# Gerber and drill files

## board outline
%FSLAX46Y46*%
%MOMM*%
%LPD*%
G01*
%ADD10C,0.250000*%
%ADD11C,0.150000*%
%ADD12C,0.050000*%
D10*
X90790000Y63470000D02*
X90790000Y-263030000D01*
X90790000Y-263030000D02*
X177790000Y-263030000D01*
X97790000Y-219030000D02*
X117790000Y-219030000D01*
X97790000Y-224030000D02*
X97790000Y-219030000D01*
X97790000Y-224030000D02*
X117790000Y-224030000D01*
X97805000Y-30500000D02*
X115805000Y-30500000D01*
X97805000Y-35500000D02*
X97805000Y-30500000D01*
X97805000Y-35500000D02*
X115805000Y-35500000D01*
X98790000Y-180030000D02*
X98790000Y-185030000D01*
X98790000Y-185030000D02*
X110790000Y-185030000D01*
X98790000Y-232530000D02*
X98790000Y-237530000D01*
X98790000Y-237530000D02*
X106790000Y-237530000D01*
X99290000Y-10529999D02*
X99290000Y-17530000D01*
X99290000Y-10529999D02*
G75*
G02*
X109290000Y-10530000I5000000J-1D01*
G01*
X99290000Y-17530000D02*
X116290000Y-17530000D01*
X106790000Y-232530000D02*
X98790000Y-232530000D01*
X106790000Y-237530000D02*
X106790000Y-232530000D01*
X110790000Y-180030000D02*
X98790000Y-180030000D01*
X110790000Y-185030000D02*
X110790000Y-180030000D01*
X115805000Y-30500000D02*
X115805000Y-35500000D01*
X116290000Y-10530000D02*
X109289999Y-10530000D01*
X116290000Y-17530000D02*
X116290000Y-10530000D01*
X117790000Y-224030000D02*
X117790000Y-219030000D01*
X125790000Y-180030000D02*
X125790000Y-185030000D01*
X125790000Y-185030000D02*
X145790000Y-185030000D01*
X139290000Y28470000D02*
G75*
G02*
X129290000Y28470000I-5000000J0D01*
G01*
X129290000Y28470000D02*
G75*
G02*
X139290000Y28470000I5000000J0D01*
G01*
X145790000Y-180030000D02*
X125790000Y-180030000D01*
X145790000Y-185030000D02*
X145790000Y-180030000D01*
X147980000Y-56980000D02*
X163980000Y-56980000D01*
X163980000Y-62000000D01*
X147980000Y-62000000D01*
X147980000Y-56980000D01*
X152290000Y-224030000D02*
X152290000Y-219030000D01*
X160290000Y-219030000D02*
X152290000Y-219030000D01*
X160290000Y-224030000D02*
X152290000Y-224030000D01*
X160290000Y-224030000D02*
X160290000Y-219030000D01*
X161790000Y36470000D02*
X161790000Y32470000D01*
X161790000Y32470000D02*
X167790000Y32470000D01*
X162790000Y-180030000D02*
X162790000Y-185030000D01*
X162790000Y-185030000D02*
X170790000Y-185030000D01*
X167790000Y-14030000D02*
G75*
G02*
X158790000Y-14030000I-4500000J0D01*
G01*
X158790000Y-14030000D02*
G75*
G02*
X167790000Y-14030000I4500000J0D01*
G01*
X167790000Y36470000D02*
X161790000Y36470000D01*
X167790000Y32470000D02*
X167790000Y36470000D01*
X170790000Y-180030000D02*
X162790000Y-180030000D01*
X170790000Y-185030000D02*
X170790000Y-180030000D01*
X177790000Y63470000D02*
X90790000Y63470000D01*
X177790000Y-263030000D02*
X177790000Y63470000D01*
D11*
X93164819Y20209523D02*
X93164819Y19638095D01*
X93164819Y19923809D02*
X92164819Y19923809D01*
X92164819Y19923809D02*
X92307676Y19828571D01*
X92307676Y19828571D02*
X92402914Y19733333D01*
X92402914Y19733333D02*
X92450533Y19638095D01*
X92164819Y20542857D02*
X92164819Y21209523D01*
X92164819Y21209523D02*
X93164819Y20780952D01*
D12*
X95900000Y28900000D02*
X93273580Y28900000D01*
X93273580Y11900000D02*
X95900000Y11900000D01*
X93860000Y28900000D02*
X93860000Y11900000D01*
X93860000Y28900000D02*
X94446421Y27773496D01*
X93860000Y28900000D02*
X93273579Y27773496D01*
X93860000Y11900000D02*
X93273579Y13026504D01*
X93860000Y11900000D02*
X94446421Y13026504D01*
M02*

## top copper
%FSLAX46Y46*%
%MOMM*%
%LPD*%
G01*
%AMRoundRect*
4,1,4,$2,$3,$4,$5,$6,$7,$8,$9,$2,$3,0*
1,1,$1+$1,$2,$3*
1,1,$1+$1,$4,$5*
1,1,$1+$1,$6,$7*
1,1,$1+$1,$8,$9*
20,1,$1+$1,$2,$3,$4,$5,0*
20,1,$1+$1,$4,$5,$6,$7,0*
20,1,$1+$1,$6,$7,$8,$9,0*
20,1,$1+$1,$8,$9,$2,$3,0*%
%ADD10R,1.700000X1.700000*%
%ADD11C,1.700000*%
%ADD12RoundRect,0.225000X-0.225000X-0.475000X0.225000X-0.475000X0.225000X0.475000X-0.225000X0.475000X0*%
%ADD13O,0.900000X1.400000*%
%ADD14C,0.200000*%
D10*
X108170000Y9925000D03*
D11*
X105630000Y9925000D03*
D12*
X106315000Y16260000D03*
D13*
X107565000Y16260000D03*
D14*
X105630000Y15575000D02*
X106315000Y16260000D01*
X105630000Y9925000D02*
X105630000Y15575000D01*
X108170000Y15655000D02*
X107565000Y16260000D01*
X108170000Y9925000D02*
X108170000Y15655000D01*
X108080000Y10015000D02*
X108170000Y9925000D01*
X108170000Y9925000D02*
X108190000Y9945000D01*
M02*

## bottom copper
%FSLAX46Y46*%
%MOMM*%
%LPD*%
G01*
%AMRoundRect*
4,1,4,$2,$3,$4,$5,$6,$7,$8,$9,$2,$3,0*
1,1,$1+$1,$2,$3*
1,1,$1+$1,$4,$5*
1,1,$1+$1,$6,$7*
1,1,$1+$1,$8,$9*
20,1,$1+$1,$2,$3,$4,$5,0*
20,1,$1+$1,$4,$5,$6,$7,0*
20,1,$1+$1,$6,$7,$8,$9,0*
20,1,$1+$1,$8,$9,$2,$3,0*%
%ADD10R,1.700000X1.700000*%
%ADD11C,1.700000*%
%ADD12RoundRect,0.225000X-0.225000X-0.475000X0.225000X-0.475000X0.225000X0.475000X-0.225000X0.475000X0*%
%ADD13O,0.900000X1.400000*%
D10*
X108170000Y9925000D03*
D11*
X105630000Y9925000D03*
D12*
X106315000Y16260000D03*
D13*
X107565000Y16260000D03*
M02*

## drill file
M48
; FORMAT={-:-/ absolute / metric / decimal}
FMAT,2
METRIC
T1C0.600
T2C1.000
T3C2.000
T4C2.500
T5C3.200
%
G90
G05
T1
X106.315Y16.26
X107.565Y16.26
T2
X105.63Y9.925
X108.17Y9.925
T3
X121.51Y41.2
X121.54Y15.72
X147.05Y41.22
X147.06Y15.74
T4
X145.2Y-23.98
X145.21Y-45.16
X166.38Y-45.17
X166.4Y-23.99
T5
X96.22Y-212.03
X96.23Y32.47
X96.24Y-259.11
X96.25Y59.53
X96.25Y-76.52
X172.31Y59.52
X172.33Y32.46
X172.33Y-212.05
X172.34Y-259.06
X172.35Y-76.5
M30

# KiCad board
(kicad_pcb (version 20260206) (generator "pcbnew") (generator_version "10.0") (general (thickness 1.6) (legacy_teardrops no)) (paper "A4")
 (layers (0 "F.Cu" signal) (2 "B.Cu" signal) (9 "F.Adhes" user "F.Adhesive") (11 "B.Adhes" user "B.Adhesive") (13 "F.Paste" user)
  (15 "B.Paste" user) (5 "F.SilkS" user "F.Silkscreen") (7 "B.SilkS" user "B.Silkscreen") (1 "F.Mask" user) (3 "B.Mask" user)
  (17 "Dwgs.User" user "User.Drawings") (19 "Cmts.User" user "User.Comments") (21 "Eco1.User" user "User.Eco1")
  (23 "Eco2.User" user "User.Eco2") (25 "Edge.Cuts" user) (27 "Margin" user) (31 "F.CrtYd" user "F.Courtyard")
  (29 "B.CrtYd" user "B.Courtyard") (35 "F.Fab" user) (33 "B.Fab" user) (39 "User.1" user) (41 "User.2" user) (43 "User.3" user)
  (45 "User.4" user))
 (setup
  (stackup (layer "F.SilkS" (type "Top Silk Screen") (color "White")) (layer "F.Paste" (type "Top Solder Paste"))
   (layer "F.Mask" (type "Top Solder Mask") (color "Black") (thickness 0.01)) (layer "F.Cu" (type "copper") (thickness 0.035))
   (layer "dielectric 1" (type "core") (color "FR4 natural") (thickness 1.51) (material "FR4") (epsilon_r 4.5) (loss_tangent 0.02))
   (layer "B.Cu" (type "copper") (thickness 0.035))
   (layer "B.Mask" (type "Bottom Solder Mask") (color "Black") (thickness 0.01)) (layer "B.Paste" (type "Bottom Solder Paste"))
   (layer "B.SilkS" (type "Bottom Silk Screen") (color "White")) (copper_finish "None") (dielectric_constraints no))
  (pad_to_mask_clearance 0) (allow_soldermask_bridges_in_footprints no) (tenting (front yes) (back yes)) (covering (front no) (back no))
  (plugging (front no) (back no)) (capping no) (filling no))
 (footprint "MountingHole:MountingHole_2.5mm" (layer "F.Cu") (at 166.4 23.99)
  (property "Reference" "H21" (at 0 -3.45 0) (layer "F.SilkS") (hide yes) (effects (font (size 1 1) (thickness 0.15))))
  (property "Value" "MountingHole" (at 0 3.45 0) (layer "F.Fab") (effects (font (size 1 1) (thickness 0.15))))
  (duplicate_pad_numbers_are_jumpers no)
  (pad "" np_thru_hole circle (at 0 0) (size 2.5 2.5) (drill 2.5) (layers "*.Cu" "*.Mask")))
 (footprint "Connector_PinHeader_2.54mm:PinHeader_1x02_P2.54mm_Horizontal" (layer "F.Cu") (at 108.17 -9.925 -90)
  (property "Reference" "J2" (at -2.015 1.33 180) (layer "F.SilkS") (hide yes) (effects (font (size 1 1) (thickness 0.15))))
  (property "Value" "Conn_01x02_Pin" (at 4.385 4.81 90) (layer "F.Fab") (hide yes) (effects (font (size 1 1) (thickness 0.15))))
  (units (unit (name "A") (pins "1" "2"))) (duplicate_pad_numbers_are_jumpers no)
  (pad "1" thru_hole rect (at 0 0 270) (size 1.7 1.7) (drill 1) (layers "*.Cu" "*.Mask") (remove_unused_layers no) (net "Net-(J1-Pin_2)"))
  (pad "2" thru_hole circle (at 0 2.54 270) (size 1.7 1.7) (drill 1) (layers "*.Cu" "*.Mask") (remove_unused_layers no)
   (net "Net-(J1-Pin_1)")))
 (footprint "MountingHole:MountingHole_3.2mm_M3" (layer "F.Cu") (at 96.25 76.52)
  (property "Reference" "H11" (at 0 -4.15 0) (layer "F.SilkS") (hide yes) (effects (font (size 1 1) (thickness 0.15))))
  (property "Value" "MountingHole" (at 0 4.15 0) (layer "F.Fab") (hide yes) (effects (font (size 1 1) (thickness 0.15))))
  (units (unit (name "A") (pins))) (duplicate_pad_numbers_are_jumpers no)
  (pad "" np_thru_hole circle (at 0 0) (size 3.2 3.2) (drill 3.2) (layers "*.Cu" "*.Mask")))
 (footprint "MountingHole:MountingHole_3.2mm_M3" (layer "F.Cu") (at 172.31 -59.52)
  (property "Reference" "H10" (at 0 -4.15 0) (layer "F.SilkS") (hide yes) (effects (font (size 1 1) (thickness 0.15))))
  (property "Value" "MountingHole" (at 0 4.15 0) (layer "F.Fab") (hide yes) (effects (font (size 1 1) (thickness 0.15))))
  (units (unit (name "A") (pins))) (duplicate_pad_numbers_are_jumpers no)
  (pad "" np_thru_hole circle (at 0 0) (size 3.2 3.2) (drill 3.2) (layers "*.Cu" "*.Mask")))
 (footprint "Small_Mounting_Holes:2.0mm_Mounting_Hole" (layer "F.Cu") (at 121.56 -15.68)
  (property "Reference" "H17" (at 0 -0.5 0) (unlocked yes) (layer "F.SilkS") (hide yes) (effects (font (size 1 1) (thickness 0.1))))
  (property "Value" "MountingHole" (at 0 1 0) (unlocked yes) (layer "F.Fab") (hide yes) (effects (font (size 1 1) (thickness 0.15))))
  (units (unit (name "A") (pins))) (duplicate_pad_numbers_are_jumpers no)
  (pad "" np_thru_hole circle (at -0.02 -0.04) (size 2 2) (drill 2) (layers "*.Cu" "*.Mask")))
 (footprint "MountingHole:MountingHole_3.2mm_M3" (layer "F.Cu") (at 96.24 259.11)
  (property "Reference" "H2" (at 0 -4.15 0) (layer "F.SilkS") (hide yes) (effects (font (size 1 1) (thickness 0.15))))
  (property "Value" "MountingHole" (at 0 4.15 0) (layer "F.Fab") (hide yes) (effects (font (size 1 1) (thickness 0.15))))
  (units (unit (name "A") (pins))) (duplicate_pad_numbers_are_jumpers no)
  (pad "" np_thru_hole circle (at 0 0) (size 3.2 3.2) (drill 3.2) (layers "*.Cu" "*.Mask")))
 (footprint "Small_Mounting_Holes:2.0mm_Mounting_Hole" (layer "F.Cu") (at 147.08 -15.7)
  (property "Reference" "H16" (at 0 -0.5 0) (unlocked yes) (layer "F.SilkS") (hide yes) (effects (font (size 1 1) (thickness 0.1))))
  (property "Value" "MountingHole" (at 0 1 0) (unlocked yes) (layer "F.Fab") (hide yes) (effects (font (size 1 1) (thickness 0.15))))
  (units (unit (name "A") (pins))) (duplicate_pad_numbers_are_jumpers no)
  (pad "" np_thru_hole circle (at -0.02 -0.04) (size 2 2) (drill 2) (layers "*.Cu" "*.Mask")))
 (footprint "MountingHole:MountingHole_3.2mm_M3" (layer "F.Cu") (at 96.23 -32.47)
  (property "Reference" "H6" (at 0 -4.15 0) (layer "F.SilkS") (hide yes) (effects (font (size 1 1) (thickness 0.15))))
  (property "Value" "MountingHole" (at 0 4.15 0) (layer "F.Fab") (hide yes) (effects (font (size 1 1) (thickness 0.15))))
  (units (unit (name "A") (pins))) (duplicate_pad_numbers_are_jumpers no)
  (pad "" np_thru_hole circle (at 0 0) (size 3.2 3.2) (drill 3.2) (layers "*.Cu" "*.Mask")))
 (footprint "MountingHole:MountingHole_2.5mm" (layer "F.Cu") (at 145.21 45.16)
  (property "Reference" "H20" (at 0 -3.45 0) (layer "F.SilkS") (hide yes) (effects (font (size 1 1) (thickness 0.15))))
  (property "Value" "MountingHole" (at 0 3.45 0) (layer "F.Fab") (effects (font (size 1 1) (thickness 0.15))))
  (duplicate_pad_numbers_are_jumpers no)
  (pad "" np_thru_hole circle (at 0 0) (size 2.5 2.5) (drill 2.5) (layers "*.Cu" "*.Mask")))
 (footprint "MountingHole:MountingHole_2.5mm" (layer "F.Cu") (at 145.2 23.98)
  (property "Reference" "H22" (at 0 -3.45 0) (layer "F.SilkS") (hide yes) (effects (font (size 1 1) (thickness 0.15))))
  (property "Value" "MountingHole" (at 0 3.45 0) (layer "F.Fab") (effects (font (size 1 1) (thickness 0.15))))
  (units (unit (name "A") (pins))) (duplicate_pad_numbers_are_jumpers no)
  (pad "" np_thru_hole circle (at 0 0) (size 2.5 2.5) (drill 2.5) (layers "*.Cu" "*.Mask")))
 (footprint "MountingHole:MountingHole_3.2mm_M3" (layer "F.Cu") (at 96.22 212.03)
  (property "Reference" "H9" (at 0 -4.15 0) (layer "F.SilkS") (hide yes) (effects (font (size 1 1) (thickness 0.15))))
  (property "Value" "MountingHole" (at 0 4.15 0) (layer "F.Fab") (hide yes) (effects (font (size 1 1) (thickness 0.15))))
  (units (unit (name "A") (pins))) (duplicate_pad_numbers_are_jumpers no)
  (pad "" np_thru_hole circle (at 0 0) (size 3.2 3.2) (drill 3.2) (layers "*.Cu" "*.Mask")))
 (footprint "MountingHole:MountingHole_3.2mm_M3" (layer "F.Cu") (at 96.25 -59.53)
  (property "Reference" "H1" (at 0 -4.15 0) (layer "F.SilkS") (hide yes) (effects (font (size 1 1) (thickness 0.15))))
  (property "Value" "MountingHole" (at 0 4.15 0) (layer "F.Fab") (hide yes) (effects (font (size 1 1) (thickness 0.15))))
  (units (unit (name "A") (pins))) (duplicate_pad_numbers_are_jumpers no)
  (pad "" np_thru_hole circle (at 0 0) (size 3.2 3.2) (drill 3.2) (layers "*.Cu" "*.Mask")))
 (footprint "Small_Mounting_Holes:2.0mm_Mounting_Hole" (layer "F.Cu") (at 147.07 -41.18)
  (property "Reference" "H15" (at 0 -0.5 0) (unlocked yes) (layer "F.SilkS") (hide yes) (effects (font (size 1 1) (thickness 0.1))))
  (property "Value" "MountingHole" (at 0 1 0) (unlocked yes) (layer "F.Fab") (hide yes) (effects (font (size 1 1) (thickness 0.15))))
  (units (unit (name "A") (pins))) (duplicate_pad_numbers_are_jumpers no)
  (pad "" np_thru_hole circle (at -0.02 -0.04) (size 2 2) (drill 2) (layers "*.Cu" "*.Mask")))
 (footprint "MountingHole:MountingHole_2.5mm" (layer "F.Cu") (at 166.38 45.17)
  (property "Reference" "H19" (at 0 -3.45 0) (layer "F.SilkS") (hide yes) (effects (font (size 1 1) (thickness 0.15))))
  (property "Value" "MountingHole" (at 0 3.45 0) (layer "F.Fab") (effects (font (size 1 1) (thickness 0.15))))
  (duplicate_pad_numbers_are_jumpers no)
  (pad "" np_thru_hole circle (at 0 0) (size 2.5 2.5) (drill 2.5) (layers "*.Cu" "*.Mask")))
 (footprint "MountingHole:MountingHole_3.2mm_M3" (layer "F.Cu") (at 172.33 212.05)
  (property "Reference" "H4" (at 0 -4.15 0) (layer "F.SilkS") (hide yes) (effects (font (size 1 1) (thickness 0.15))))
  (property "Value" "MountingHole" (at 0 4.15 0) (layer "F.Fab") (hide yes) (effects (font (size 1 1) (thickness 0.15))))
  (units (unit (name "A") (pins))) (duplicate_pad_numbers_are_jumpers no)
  (pad "" np_thru_hole circle (at 0 0) (size 3.2 3.2) (drill 3.2) (layers "*.Cu" "*.Mask")))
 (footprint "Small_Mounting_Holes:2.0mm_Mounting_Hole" (layer "F.Cu") (at 121.53 -41.16)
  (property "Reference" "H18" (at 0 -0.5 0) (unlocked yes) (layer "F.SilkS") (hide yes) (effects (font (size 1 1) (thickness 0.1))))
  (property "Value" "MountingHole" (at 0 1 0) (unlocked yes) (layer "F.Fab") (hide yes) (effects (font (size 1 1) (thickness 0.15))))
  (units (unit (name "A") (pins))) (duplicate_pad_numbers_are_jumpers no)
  (pad "" np_thru_hole circle (at -0.02 -0.04) (size 2 2) (drill 2) (layers "*.Cu" "*.Mask")))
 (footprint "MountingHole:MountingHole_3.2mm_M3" (layer "F.Cu") (at 172.33 -32.46)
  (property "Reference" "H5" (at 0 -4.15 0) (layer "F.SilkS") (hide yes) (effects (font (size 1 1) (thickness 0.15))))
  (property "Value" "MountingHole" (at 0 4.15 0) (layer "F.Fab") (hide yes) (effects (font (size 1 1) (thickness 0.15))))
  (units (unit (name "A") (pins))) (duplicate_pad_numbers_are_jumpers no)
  (pad "" np_thru_hole circle (at 0 0) (size 3.2 3.2) (drill 3.2) (layers "*.Cu" "*.Mask")))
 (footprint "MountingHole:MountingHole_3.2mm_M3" (layer "F.Cu") (at 172.35 76.5)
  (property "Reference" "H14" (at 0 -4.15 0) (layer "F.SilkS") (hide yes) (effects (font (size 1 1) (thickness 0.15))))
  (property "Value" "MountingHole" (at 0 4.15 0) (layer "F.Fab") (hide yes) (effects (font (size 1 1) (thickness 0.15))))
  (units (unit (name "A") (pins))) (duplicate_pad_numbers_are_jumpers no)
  (pad "" np_thru_hole circle (at 0 0) (size 3.2 3.2) (drill 3.2) (layers "*.Cu" "*.Mask")))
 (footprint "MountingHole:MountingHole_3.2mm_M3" (layer "F.Cu") (at 172.34 259.06)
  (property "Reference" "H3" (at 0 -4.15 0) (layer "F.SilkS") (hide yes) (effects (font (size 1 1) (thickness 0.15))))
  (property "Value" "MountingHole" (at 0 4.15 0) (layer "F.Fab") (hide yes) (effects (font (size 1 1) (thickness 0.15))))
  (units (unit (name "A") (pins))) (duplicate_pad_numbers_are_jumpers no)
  (pad "" np_thru_hole circle (at 0 0) (size 3.2 3.2) (drill 3.2) (layers "*.Cu" "*.Mask")))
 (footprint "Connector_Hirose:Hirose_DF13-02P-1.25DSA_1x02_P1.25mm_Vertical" (layer "B.Cu") (at 106.315 -16.26)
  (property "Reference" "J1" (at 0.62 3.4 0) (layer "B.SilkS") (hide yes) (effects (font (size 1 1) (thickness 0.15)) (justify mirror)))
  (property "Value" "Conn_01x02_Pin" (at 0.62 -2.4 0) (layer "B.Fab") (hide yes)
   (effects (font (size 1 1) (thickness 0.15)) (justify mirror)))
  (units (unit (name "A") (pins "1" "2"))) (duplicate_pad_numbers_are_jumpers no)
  (pad "1" thru_hole roundrect (at 0 0) (size 0.9 1.4) (drill 0.6) (layers "*.Cu" "*.Mask") (remove_unused_layers no)
   (roundrect_rratio 0.25) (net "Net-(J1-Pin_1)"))
  (pad "2" thru_hole oval (at 1.25 0) (size 0.9 1.4) (drill 0.6) (layers "*.Cu" "*.Mask") (remove_unused_layers no) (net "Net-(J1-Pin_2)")))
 (gr_line (start 90.79 -63.47) (end 90.79 263.03) (stroke (width 0.25) (type default)) (layer "Edge.Cuts"))
 (gr_line (start 90.79 263.03) (end 177.79 263.03) (stroke (width 0.25) (type default)) (layer "Edge.Cuts"))
 (gr_line (start 97.79 219.03) (end 117.79 219.03) (stroke (width 0.25) (type default)) (layer "Edge.Cuts"))
 (gr_line (start 97.79 224.03) (end 97.79 219.03) (stroke (width 0.25) (type default)) (layer "Edge.Cuts"))
 (gr_line (start 97.79 224.03) (end 117.79 224.03) (stroke (width 0.25) (type default)) (layer "Edge.Cuts"))
 (gr_line (start 97.805 30.5) (end 115.805 30.5) (stroke (width 0.25) (type solid)) (layer "Edge.Cuts"))
 (gr_line (start 97.805 35.5) (end 97.805 30.5) (stroke (width 0.25) (type solid)) (layer "Edge.Cuts"))
 (gr_line (start 97.805 35.5) (end 115.805 35.5) (stroke (width 0.25) (type solid)) (layer "Edge.Cuts"))
 (gr_line (start 98.79 180.03) (end 98.79 185.03) (stroke (width 0.25) (type default)) (layer "Edge.Cuts"))
 (gr_line (start 98.79 185.03) (end 110.79 185.03) (stroke (width 0.25) (type default)) (layer "Edge.Cuts"))
 (gr_line (start 98.79 232.53) (end 98.79 237.53) (stroke (width 0.25) (type default)) (layer "Edge.Cuts"))
 (gr_line (start 98.79 237.53) (end 106.79 237.53) (stroke (width 0.25) (type default)) (layer "Edge.Cuts"))
 (gr_line (start 99.29 10.529999) (end 99.29 17.53) (stroke (width 0.25) (type default)) (layer "Edge.Cuts"))
 (gr_arc (start 99.29 10.529999) (mid 104.29 5.53) (end 109.289999 10.53) (stroke (width 0.25) (type default)) (layer "Edge.Cuts"))
 (gr_line (start 99.29 17.53) (end 116.29 17.53) (stroke (width 0.25) (type default)) (layer "Edge.Cuts"))
 (gr_line (start 106.79 232.53) (end 98.79 232.53) (stroke (width 0.25) (type default)) (layer "Edge.Cuts"))
 (gr_line (start 106.79 237.53) (end 106.79 232.53) (stroke (width 0.25) (type default)) (layer "Edge.Cuts"))
 (gr_line (start 110.79 180.03) (end 98.79 180.03) (stroke (width 0.25) (type default)) (layer "Edge.Cuts"))
 (gr_line (start 110.79 185.03) (end 110.79 180.03) (stroke (width 0.25) (type default)) (layer "Edge.Cuts"))
 (gr_line (start 115.805 30.5) (end 115.805 35.5) (stroke (width 0.25) (type solid)) (layer "Edge.Cuts"))
 (gr_line (start 116.29 10.53) (end 109.289999 10.53) (stroke (width 0.25) (type default)) (layer "Edge.Cuts"))
 (gr_line (start 116.29 17.53) (end 116.29 10.53) (stroke (width 0.25) (type default)) (layer "Edge.Cuts"))
 (gr_line (start 117.79 224.03) (end 117.79 219.03) (stroke (width 0.25) (type default)) (layer "Edge.Cuts"))
 (gr_line (start 125.79 180.03) (end 125.79 185.03) (stroke (width 0.25) (type default)) (layer "Edge.Cuts"))
 (gr_line (start 125.79 185.03) (end 145.79 185.03) (stroke (width 0.25) (type default)) (layer "Edge.Cuts"))
 (gr_circle (center 134.29 -28.47) (end 139.29 -28.47) (stroke (width 0.25) (type default)) (fill no) (layer "Edge.Cuts"))
 (gr_line (start 145.79 180.03) (end 125.79 180.03) (stroke (width 0.25) (type solid)) (layer "Edge.Cuts"))
 (gr_line (start 145.79 185.03) (end 145.79 180.03) (stroke (width 0.25) (type default)) (layer "Edge.Cuts"))
 (gr_rect (start 147.98 56.98) (end 163.98 62) (stroke (width 0.25) (type solid)) (fill no) (layer "Edge.Cuts"))
 (gr_line (start 152.29 224.03) (end 152.29 219.03) (stroke (width 0.25) (type default)) (layer "Edge.Cuts"))
 (gr_line (start 160.29 219.03) (end 152.29 219.03) (stroke (width 0.25) (type default)) (layer "Edge.Cuts"))
 (gr_line (start 160.29 224.03) (end 152.29 224.03) (stroke (width 0.25) (type default)) (layer "Edge.Cuts"))
 (gr_line (start 160.29 224.03) (end 160.29 219.03) (stroke (width 0.25) (type default)) (layer "Edge.Cuts"))
 (gr_line (start 161.79 -36.47) (end 161.79 -32.47) (stroke (width 0.25) (type default)) (layer "Edge.Cuts"))
 (gr_line (start 161.79 -32.47) (end 167.79 -32.47) (stroke (width 0.25) (type default)) (layer "Edge.Cuts"))
 (gr_line (start 162.79 180.03) (end 162.79 185.03) (stroke (width 0.25) (type default)) (layer "Edge.Cuts"))
 (gr_line (start 162.79 185.03) (end 170.79 185.03) (stroke (width 0.25) (type default)) (layer "Edge.Cuts"))
 (gr_circle (center 163.29 14.03) (end 167.79 14.03) (stroke (width 0.25) (type default)) (fill no) (layer "Edge.Cuts"))
 (gr_line (start 167.79 -36.47) (end 161.79 -36.47) (stroke (width 0.25) (type default)) (layer "Edge.Cuts"))
 (gr_line (start 167.79 -32.47) (end 167.79 -36.47) (stroke (width 0.25) (type default)) (layer "Edge.Cuts"))
 (gr_line (start 170.79 180.03) (end 162.79 180.03) (stroke (width 0.25) (type default)) (layer "Edge.Cuts"))
 (gr_line (start 170.79 185.03) (end 170.79 180.03) (stroke (width 0.25) (type default)) (layer "Edge.Cuts"))
 (gr_line (start 177.79 -63.47) (end 90.79 -63.47) (stroke (width 0.25) (type default)) (layer "Edge.Cuts"))
 (gr_line (start 177.79 263.03) (end 177.79 -63.47) (stroke (width 0.25) (type default)) (layer "Edge.Cuts"))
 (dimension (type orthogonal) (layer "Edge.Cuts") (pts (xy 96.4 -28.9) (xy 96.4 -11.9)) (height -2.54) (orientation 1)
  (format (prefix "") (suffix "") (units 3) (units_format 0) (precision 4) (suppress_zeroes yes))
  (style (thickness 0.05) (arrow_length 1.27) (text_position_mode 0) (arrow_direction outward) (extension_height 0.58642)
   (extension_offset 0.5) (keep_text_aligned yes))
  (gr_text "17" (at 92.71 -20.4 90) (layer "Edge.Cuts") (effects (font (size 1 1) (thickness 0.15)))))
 (segment (start 105.63 -15.575) (end 106.315 -16.26) (width 0.2) (layer "F.Cu") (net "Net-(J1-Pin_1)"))
 (segment (start 105.63 -9.925) (end 105.63 -15.575) (width 0.2) (layer "F.Cu") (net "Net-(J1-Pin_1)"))
 (segment (start 108.17 -15.655) (end 107.565 -16.26) (width 0.2) (layer "F.Cu") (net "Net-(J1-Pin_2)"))
 (segment (start 108.17 -9.925) (end 108.17 -15.655) (width 0.2) (layer "F.Cu") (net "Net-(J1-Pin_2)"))
 (segment (start 108.08 -10.015) (end 108.17 -9.925) (width 0.2) (layer "F.Cu") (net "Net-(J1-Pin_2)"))
 (segment (start 108.17 -9.925) (end 108.19 -9.945) (width 0.2) (layer "F.Cu") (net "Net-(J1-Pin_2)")))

